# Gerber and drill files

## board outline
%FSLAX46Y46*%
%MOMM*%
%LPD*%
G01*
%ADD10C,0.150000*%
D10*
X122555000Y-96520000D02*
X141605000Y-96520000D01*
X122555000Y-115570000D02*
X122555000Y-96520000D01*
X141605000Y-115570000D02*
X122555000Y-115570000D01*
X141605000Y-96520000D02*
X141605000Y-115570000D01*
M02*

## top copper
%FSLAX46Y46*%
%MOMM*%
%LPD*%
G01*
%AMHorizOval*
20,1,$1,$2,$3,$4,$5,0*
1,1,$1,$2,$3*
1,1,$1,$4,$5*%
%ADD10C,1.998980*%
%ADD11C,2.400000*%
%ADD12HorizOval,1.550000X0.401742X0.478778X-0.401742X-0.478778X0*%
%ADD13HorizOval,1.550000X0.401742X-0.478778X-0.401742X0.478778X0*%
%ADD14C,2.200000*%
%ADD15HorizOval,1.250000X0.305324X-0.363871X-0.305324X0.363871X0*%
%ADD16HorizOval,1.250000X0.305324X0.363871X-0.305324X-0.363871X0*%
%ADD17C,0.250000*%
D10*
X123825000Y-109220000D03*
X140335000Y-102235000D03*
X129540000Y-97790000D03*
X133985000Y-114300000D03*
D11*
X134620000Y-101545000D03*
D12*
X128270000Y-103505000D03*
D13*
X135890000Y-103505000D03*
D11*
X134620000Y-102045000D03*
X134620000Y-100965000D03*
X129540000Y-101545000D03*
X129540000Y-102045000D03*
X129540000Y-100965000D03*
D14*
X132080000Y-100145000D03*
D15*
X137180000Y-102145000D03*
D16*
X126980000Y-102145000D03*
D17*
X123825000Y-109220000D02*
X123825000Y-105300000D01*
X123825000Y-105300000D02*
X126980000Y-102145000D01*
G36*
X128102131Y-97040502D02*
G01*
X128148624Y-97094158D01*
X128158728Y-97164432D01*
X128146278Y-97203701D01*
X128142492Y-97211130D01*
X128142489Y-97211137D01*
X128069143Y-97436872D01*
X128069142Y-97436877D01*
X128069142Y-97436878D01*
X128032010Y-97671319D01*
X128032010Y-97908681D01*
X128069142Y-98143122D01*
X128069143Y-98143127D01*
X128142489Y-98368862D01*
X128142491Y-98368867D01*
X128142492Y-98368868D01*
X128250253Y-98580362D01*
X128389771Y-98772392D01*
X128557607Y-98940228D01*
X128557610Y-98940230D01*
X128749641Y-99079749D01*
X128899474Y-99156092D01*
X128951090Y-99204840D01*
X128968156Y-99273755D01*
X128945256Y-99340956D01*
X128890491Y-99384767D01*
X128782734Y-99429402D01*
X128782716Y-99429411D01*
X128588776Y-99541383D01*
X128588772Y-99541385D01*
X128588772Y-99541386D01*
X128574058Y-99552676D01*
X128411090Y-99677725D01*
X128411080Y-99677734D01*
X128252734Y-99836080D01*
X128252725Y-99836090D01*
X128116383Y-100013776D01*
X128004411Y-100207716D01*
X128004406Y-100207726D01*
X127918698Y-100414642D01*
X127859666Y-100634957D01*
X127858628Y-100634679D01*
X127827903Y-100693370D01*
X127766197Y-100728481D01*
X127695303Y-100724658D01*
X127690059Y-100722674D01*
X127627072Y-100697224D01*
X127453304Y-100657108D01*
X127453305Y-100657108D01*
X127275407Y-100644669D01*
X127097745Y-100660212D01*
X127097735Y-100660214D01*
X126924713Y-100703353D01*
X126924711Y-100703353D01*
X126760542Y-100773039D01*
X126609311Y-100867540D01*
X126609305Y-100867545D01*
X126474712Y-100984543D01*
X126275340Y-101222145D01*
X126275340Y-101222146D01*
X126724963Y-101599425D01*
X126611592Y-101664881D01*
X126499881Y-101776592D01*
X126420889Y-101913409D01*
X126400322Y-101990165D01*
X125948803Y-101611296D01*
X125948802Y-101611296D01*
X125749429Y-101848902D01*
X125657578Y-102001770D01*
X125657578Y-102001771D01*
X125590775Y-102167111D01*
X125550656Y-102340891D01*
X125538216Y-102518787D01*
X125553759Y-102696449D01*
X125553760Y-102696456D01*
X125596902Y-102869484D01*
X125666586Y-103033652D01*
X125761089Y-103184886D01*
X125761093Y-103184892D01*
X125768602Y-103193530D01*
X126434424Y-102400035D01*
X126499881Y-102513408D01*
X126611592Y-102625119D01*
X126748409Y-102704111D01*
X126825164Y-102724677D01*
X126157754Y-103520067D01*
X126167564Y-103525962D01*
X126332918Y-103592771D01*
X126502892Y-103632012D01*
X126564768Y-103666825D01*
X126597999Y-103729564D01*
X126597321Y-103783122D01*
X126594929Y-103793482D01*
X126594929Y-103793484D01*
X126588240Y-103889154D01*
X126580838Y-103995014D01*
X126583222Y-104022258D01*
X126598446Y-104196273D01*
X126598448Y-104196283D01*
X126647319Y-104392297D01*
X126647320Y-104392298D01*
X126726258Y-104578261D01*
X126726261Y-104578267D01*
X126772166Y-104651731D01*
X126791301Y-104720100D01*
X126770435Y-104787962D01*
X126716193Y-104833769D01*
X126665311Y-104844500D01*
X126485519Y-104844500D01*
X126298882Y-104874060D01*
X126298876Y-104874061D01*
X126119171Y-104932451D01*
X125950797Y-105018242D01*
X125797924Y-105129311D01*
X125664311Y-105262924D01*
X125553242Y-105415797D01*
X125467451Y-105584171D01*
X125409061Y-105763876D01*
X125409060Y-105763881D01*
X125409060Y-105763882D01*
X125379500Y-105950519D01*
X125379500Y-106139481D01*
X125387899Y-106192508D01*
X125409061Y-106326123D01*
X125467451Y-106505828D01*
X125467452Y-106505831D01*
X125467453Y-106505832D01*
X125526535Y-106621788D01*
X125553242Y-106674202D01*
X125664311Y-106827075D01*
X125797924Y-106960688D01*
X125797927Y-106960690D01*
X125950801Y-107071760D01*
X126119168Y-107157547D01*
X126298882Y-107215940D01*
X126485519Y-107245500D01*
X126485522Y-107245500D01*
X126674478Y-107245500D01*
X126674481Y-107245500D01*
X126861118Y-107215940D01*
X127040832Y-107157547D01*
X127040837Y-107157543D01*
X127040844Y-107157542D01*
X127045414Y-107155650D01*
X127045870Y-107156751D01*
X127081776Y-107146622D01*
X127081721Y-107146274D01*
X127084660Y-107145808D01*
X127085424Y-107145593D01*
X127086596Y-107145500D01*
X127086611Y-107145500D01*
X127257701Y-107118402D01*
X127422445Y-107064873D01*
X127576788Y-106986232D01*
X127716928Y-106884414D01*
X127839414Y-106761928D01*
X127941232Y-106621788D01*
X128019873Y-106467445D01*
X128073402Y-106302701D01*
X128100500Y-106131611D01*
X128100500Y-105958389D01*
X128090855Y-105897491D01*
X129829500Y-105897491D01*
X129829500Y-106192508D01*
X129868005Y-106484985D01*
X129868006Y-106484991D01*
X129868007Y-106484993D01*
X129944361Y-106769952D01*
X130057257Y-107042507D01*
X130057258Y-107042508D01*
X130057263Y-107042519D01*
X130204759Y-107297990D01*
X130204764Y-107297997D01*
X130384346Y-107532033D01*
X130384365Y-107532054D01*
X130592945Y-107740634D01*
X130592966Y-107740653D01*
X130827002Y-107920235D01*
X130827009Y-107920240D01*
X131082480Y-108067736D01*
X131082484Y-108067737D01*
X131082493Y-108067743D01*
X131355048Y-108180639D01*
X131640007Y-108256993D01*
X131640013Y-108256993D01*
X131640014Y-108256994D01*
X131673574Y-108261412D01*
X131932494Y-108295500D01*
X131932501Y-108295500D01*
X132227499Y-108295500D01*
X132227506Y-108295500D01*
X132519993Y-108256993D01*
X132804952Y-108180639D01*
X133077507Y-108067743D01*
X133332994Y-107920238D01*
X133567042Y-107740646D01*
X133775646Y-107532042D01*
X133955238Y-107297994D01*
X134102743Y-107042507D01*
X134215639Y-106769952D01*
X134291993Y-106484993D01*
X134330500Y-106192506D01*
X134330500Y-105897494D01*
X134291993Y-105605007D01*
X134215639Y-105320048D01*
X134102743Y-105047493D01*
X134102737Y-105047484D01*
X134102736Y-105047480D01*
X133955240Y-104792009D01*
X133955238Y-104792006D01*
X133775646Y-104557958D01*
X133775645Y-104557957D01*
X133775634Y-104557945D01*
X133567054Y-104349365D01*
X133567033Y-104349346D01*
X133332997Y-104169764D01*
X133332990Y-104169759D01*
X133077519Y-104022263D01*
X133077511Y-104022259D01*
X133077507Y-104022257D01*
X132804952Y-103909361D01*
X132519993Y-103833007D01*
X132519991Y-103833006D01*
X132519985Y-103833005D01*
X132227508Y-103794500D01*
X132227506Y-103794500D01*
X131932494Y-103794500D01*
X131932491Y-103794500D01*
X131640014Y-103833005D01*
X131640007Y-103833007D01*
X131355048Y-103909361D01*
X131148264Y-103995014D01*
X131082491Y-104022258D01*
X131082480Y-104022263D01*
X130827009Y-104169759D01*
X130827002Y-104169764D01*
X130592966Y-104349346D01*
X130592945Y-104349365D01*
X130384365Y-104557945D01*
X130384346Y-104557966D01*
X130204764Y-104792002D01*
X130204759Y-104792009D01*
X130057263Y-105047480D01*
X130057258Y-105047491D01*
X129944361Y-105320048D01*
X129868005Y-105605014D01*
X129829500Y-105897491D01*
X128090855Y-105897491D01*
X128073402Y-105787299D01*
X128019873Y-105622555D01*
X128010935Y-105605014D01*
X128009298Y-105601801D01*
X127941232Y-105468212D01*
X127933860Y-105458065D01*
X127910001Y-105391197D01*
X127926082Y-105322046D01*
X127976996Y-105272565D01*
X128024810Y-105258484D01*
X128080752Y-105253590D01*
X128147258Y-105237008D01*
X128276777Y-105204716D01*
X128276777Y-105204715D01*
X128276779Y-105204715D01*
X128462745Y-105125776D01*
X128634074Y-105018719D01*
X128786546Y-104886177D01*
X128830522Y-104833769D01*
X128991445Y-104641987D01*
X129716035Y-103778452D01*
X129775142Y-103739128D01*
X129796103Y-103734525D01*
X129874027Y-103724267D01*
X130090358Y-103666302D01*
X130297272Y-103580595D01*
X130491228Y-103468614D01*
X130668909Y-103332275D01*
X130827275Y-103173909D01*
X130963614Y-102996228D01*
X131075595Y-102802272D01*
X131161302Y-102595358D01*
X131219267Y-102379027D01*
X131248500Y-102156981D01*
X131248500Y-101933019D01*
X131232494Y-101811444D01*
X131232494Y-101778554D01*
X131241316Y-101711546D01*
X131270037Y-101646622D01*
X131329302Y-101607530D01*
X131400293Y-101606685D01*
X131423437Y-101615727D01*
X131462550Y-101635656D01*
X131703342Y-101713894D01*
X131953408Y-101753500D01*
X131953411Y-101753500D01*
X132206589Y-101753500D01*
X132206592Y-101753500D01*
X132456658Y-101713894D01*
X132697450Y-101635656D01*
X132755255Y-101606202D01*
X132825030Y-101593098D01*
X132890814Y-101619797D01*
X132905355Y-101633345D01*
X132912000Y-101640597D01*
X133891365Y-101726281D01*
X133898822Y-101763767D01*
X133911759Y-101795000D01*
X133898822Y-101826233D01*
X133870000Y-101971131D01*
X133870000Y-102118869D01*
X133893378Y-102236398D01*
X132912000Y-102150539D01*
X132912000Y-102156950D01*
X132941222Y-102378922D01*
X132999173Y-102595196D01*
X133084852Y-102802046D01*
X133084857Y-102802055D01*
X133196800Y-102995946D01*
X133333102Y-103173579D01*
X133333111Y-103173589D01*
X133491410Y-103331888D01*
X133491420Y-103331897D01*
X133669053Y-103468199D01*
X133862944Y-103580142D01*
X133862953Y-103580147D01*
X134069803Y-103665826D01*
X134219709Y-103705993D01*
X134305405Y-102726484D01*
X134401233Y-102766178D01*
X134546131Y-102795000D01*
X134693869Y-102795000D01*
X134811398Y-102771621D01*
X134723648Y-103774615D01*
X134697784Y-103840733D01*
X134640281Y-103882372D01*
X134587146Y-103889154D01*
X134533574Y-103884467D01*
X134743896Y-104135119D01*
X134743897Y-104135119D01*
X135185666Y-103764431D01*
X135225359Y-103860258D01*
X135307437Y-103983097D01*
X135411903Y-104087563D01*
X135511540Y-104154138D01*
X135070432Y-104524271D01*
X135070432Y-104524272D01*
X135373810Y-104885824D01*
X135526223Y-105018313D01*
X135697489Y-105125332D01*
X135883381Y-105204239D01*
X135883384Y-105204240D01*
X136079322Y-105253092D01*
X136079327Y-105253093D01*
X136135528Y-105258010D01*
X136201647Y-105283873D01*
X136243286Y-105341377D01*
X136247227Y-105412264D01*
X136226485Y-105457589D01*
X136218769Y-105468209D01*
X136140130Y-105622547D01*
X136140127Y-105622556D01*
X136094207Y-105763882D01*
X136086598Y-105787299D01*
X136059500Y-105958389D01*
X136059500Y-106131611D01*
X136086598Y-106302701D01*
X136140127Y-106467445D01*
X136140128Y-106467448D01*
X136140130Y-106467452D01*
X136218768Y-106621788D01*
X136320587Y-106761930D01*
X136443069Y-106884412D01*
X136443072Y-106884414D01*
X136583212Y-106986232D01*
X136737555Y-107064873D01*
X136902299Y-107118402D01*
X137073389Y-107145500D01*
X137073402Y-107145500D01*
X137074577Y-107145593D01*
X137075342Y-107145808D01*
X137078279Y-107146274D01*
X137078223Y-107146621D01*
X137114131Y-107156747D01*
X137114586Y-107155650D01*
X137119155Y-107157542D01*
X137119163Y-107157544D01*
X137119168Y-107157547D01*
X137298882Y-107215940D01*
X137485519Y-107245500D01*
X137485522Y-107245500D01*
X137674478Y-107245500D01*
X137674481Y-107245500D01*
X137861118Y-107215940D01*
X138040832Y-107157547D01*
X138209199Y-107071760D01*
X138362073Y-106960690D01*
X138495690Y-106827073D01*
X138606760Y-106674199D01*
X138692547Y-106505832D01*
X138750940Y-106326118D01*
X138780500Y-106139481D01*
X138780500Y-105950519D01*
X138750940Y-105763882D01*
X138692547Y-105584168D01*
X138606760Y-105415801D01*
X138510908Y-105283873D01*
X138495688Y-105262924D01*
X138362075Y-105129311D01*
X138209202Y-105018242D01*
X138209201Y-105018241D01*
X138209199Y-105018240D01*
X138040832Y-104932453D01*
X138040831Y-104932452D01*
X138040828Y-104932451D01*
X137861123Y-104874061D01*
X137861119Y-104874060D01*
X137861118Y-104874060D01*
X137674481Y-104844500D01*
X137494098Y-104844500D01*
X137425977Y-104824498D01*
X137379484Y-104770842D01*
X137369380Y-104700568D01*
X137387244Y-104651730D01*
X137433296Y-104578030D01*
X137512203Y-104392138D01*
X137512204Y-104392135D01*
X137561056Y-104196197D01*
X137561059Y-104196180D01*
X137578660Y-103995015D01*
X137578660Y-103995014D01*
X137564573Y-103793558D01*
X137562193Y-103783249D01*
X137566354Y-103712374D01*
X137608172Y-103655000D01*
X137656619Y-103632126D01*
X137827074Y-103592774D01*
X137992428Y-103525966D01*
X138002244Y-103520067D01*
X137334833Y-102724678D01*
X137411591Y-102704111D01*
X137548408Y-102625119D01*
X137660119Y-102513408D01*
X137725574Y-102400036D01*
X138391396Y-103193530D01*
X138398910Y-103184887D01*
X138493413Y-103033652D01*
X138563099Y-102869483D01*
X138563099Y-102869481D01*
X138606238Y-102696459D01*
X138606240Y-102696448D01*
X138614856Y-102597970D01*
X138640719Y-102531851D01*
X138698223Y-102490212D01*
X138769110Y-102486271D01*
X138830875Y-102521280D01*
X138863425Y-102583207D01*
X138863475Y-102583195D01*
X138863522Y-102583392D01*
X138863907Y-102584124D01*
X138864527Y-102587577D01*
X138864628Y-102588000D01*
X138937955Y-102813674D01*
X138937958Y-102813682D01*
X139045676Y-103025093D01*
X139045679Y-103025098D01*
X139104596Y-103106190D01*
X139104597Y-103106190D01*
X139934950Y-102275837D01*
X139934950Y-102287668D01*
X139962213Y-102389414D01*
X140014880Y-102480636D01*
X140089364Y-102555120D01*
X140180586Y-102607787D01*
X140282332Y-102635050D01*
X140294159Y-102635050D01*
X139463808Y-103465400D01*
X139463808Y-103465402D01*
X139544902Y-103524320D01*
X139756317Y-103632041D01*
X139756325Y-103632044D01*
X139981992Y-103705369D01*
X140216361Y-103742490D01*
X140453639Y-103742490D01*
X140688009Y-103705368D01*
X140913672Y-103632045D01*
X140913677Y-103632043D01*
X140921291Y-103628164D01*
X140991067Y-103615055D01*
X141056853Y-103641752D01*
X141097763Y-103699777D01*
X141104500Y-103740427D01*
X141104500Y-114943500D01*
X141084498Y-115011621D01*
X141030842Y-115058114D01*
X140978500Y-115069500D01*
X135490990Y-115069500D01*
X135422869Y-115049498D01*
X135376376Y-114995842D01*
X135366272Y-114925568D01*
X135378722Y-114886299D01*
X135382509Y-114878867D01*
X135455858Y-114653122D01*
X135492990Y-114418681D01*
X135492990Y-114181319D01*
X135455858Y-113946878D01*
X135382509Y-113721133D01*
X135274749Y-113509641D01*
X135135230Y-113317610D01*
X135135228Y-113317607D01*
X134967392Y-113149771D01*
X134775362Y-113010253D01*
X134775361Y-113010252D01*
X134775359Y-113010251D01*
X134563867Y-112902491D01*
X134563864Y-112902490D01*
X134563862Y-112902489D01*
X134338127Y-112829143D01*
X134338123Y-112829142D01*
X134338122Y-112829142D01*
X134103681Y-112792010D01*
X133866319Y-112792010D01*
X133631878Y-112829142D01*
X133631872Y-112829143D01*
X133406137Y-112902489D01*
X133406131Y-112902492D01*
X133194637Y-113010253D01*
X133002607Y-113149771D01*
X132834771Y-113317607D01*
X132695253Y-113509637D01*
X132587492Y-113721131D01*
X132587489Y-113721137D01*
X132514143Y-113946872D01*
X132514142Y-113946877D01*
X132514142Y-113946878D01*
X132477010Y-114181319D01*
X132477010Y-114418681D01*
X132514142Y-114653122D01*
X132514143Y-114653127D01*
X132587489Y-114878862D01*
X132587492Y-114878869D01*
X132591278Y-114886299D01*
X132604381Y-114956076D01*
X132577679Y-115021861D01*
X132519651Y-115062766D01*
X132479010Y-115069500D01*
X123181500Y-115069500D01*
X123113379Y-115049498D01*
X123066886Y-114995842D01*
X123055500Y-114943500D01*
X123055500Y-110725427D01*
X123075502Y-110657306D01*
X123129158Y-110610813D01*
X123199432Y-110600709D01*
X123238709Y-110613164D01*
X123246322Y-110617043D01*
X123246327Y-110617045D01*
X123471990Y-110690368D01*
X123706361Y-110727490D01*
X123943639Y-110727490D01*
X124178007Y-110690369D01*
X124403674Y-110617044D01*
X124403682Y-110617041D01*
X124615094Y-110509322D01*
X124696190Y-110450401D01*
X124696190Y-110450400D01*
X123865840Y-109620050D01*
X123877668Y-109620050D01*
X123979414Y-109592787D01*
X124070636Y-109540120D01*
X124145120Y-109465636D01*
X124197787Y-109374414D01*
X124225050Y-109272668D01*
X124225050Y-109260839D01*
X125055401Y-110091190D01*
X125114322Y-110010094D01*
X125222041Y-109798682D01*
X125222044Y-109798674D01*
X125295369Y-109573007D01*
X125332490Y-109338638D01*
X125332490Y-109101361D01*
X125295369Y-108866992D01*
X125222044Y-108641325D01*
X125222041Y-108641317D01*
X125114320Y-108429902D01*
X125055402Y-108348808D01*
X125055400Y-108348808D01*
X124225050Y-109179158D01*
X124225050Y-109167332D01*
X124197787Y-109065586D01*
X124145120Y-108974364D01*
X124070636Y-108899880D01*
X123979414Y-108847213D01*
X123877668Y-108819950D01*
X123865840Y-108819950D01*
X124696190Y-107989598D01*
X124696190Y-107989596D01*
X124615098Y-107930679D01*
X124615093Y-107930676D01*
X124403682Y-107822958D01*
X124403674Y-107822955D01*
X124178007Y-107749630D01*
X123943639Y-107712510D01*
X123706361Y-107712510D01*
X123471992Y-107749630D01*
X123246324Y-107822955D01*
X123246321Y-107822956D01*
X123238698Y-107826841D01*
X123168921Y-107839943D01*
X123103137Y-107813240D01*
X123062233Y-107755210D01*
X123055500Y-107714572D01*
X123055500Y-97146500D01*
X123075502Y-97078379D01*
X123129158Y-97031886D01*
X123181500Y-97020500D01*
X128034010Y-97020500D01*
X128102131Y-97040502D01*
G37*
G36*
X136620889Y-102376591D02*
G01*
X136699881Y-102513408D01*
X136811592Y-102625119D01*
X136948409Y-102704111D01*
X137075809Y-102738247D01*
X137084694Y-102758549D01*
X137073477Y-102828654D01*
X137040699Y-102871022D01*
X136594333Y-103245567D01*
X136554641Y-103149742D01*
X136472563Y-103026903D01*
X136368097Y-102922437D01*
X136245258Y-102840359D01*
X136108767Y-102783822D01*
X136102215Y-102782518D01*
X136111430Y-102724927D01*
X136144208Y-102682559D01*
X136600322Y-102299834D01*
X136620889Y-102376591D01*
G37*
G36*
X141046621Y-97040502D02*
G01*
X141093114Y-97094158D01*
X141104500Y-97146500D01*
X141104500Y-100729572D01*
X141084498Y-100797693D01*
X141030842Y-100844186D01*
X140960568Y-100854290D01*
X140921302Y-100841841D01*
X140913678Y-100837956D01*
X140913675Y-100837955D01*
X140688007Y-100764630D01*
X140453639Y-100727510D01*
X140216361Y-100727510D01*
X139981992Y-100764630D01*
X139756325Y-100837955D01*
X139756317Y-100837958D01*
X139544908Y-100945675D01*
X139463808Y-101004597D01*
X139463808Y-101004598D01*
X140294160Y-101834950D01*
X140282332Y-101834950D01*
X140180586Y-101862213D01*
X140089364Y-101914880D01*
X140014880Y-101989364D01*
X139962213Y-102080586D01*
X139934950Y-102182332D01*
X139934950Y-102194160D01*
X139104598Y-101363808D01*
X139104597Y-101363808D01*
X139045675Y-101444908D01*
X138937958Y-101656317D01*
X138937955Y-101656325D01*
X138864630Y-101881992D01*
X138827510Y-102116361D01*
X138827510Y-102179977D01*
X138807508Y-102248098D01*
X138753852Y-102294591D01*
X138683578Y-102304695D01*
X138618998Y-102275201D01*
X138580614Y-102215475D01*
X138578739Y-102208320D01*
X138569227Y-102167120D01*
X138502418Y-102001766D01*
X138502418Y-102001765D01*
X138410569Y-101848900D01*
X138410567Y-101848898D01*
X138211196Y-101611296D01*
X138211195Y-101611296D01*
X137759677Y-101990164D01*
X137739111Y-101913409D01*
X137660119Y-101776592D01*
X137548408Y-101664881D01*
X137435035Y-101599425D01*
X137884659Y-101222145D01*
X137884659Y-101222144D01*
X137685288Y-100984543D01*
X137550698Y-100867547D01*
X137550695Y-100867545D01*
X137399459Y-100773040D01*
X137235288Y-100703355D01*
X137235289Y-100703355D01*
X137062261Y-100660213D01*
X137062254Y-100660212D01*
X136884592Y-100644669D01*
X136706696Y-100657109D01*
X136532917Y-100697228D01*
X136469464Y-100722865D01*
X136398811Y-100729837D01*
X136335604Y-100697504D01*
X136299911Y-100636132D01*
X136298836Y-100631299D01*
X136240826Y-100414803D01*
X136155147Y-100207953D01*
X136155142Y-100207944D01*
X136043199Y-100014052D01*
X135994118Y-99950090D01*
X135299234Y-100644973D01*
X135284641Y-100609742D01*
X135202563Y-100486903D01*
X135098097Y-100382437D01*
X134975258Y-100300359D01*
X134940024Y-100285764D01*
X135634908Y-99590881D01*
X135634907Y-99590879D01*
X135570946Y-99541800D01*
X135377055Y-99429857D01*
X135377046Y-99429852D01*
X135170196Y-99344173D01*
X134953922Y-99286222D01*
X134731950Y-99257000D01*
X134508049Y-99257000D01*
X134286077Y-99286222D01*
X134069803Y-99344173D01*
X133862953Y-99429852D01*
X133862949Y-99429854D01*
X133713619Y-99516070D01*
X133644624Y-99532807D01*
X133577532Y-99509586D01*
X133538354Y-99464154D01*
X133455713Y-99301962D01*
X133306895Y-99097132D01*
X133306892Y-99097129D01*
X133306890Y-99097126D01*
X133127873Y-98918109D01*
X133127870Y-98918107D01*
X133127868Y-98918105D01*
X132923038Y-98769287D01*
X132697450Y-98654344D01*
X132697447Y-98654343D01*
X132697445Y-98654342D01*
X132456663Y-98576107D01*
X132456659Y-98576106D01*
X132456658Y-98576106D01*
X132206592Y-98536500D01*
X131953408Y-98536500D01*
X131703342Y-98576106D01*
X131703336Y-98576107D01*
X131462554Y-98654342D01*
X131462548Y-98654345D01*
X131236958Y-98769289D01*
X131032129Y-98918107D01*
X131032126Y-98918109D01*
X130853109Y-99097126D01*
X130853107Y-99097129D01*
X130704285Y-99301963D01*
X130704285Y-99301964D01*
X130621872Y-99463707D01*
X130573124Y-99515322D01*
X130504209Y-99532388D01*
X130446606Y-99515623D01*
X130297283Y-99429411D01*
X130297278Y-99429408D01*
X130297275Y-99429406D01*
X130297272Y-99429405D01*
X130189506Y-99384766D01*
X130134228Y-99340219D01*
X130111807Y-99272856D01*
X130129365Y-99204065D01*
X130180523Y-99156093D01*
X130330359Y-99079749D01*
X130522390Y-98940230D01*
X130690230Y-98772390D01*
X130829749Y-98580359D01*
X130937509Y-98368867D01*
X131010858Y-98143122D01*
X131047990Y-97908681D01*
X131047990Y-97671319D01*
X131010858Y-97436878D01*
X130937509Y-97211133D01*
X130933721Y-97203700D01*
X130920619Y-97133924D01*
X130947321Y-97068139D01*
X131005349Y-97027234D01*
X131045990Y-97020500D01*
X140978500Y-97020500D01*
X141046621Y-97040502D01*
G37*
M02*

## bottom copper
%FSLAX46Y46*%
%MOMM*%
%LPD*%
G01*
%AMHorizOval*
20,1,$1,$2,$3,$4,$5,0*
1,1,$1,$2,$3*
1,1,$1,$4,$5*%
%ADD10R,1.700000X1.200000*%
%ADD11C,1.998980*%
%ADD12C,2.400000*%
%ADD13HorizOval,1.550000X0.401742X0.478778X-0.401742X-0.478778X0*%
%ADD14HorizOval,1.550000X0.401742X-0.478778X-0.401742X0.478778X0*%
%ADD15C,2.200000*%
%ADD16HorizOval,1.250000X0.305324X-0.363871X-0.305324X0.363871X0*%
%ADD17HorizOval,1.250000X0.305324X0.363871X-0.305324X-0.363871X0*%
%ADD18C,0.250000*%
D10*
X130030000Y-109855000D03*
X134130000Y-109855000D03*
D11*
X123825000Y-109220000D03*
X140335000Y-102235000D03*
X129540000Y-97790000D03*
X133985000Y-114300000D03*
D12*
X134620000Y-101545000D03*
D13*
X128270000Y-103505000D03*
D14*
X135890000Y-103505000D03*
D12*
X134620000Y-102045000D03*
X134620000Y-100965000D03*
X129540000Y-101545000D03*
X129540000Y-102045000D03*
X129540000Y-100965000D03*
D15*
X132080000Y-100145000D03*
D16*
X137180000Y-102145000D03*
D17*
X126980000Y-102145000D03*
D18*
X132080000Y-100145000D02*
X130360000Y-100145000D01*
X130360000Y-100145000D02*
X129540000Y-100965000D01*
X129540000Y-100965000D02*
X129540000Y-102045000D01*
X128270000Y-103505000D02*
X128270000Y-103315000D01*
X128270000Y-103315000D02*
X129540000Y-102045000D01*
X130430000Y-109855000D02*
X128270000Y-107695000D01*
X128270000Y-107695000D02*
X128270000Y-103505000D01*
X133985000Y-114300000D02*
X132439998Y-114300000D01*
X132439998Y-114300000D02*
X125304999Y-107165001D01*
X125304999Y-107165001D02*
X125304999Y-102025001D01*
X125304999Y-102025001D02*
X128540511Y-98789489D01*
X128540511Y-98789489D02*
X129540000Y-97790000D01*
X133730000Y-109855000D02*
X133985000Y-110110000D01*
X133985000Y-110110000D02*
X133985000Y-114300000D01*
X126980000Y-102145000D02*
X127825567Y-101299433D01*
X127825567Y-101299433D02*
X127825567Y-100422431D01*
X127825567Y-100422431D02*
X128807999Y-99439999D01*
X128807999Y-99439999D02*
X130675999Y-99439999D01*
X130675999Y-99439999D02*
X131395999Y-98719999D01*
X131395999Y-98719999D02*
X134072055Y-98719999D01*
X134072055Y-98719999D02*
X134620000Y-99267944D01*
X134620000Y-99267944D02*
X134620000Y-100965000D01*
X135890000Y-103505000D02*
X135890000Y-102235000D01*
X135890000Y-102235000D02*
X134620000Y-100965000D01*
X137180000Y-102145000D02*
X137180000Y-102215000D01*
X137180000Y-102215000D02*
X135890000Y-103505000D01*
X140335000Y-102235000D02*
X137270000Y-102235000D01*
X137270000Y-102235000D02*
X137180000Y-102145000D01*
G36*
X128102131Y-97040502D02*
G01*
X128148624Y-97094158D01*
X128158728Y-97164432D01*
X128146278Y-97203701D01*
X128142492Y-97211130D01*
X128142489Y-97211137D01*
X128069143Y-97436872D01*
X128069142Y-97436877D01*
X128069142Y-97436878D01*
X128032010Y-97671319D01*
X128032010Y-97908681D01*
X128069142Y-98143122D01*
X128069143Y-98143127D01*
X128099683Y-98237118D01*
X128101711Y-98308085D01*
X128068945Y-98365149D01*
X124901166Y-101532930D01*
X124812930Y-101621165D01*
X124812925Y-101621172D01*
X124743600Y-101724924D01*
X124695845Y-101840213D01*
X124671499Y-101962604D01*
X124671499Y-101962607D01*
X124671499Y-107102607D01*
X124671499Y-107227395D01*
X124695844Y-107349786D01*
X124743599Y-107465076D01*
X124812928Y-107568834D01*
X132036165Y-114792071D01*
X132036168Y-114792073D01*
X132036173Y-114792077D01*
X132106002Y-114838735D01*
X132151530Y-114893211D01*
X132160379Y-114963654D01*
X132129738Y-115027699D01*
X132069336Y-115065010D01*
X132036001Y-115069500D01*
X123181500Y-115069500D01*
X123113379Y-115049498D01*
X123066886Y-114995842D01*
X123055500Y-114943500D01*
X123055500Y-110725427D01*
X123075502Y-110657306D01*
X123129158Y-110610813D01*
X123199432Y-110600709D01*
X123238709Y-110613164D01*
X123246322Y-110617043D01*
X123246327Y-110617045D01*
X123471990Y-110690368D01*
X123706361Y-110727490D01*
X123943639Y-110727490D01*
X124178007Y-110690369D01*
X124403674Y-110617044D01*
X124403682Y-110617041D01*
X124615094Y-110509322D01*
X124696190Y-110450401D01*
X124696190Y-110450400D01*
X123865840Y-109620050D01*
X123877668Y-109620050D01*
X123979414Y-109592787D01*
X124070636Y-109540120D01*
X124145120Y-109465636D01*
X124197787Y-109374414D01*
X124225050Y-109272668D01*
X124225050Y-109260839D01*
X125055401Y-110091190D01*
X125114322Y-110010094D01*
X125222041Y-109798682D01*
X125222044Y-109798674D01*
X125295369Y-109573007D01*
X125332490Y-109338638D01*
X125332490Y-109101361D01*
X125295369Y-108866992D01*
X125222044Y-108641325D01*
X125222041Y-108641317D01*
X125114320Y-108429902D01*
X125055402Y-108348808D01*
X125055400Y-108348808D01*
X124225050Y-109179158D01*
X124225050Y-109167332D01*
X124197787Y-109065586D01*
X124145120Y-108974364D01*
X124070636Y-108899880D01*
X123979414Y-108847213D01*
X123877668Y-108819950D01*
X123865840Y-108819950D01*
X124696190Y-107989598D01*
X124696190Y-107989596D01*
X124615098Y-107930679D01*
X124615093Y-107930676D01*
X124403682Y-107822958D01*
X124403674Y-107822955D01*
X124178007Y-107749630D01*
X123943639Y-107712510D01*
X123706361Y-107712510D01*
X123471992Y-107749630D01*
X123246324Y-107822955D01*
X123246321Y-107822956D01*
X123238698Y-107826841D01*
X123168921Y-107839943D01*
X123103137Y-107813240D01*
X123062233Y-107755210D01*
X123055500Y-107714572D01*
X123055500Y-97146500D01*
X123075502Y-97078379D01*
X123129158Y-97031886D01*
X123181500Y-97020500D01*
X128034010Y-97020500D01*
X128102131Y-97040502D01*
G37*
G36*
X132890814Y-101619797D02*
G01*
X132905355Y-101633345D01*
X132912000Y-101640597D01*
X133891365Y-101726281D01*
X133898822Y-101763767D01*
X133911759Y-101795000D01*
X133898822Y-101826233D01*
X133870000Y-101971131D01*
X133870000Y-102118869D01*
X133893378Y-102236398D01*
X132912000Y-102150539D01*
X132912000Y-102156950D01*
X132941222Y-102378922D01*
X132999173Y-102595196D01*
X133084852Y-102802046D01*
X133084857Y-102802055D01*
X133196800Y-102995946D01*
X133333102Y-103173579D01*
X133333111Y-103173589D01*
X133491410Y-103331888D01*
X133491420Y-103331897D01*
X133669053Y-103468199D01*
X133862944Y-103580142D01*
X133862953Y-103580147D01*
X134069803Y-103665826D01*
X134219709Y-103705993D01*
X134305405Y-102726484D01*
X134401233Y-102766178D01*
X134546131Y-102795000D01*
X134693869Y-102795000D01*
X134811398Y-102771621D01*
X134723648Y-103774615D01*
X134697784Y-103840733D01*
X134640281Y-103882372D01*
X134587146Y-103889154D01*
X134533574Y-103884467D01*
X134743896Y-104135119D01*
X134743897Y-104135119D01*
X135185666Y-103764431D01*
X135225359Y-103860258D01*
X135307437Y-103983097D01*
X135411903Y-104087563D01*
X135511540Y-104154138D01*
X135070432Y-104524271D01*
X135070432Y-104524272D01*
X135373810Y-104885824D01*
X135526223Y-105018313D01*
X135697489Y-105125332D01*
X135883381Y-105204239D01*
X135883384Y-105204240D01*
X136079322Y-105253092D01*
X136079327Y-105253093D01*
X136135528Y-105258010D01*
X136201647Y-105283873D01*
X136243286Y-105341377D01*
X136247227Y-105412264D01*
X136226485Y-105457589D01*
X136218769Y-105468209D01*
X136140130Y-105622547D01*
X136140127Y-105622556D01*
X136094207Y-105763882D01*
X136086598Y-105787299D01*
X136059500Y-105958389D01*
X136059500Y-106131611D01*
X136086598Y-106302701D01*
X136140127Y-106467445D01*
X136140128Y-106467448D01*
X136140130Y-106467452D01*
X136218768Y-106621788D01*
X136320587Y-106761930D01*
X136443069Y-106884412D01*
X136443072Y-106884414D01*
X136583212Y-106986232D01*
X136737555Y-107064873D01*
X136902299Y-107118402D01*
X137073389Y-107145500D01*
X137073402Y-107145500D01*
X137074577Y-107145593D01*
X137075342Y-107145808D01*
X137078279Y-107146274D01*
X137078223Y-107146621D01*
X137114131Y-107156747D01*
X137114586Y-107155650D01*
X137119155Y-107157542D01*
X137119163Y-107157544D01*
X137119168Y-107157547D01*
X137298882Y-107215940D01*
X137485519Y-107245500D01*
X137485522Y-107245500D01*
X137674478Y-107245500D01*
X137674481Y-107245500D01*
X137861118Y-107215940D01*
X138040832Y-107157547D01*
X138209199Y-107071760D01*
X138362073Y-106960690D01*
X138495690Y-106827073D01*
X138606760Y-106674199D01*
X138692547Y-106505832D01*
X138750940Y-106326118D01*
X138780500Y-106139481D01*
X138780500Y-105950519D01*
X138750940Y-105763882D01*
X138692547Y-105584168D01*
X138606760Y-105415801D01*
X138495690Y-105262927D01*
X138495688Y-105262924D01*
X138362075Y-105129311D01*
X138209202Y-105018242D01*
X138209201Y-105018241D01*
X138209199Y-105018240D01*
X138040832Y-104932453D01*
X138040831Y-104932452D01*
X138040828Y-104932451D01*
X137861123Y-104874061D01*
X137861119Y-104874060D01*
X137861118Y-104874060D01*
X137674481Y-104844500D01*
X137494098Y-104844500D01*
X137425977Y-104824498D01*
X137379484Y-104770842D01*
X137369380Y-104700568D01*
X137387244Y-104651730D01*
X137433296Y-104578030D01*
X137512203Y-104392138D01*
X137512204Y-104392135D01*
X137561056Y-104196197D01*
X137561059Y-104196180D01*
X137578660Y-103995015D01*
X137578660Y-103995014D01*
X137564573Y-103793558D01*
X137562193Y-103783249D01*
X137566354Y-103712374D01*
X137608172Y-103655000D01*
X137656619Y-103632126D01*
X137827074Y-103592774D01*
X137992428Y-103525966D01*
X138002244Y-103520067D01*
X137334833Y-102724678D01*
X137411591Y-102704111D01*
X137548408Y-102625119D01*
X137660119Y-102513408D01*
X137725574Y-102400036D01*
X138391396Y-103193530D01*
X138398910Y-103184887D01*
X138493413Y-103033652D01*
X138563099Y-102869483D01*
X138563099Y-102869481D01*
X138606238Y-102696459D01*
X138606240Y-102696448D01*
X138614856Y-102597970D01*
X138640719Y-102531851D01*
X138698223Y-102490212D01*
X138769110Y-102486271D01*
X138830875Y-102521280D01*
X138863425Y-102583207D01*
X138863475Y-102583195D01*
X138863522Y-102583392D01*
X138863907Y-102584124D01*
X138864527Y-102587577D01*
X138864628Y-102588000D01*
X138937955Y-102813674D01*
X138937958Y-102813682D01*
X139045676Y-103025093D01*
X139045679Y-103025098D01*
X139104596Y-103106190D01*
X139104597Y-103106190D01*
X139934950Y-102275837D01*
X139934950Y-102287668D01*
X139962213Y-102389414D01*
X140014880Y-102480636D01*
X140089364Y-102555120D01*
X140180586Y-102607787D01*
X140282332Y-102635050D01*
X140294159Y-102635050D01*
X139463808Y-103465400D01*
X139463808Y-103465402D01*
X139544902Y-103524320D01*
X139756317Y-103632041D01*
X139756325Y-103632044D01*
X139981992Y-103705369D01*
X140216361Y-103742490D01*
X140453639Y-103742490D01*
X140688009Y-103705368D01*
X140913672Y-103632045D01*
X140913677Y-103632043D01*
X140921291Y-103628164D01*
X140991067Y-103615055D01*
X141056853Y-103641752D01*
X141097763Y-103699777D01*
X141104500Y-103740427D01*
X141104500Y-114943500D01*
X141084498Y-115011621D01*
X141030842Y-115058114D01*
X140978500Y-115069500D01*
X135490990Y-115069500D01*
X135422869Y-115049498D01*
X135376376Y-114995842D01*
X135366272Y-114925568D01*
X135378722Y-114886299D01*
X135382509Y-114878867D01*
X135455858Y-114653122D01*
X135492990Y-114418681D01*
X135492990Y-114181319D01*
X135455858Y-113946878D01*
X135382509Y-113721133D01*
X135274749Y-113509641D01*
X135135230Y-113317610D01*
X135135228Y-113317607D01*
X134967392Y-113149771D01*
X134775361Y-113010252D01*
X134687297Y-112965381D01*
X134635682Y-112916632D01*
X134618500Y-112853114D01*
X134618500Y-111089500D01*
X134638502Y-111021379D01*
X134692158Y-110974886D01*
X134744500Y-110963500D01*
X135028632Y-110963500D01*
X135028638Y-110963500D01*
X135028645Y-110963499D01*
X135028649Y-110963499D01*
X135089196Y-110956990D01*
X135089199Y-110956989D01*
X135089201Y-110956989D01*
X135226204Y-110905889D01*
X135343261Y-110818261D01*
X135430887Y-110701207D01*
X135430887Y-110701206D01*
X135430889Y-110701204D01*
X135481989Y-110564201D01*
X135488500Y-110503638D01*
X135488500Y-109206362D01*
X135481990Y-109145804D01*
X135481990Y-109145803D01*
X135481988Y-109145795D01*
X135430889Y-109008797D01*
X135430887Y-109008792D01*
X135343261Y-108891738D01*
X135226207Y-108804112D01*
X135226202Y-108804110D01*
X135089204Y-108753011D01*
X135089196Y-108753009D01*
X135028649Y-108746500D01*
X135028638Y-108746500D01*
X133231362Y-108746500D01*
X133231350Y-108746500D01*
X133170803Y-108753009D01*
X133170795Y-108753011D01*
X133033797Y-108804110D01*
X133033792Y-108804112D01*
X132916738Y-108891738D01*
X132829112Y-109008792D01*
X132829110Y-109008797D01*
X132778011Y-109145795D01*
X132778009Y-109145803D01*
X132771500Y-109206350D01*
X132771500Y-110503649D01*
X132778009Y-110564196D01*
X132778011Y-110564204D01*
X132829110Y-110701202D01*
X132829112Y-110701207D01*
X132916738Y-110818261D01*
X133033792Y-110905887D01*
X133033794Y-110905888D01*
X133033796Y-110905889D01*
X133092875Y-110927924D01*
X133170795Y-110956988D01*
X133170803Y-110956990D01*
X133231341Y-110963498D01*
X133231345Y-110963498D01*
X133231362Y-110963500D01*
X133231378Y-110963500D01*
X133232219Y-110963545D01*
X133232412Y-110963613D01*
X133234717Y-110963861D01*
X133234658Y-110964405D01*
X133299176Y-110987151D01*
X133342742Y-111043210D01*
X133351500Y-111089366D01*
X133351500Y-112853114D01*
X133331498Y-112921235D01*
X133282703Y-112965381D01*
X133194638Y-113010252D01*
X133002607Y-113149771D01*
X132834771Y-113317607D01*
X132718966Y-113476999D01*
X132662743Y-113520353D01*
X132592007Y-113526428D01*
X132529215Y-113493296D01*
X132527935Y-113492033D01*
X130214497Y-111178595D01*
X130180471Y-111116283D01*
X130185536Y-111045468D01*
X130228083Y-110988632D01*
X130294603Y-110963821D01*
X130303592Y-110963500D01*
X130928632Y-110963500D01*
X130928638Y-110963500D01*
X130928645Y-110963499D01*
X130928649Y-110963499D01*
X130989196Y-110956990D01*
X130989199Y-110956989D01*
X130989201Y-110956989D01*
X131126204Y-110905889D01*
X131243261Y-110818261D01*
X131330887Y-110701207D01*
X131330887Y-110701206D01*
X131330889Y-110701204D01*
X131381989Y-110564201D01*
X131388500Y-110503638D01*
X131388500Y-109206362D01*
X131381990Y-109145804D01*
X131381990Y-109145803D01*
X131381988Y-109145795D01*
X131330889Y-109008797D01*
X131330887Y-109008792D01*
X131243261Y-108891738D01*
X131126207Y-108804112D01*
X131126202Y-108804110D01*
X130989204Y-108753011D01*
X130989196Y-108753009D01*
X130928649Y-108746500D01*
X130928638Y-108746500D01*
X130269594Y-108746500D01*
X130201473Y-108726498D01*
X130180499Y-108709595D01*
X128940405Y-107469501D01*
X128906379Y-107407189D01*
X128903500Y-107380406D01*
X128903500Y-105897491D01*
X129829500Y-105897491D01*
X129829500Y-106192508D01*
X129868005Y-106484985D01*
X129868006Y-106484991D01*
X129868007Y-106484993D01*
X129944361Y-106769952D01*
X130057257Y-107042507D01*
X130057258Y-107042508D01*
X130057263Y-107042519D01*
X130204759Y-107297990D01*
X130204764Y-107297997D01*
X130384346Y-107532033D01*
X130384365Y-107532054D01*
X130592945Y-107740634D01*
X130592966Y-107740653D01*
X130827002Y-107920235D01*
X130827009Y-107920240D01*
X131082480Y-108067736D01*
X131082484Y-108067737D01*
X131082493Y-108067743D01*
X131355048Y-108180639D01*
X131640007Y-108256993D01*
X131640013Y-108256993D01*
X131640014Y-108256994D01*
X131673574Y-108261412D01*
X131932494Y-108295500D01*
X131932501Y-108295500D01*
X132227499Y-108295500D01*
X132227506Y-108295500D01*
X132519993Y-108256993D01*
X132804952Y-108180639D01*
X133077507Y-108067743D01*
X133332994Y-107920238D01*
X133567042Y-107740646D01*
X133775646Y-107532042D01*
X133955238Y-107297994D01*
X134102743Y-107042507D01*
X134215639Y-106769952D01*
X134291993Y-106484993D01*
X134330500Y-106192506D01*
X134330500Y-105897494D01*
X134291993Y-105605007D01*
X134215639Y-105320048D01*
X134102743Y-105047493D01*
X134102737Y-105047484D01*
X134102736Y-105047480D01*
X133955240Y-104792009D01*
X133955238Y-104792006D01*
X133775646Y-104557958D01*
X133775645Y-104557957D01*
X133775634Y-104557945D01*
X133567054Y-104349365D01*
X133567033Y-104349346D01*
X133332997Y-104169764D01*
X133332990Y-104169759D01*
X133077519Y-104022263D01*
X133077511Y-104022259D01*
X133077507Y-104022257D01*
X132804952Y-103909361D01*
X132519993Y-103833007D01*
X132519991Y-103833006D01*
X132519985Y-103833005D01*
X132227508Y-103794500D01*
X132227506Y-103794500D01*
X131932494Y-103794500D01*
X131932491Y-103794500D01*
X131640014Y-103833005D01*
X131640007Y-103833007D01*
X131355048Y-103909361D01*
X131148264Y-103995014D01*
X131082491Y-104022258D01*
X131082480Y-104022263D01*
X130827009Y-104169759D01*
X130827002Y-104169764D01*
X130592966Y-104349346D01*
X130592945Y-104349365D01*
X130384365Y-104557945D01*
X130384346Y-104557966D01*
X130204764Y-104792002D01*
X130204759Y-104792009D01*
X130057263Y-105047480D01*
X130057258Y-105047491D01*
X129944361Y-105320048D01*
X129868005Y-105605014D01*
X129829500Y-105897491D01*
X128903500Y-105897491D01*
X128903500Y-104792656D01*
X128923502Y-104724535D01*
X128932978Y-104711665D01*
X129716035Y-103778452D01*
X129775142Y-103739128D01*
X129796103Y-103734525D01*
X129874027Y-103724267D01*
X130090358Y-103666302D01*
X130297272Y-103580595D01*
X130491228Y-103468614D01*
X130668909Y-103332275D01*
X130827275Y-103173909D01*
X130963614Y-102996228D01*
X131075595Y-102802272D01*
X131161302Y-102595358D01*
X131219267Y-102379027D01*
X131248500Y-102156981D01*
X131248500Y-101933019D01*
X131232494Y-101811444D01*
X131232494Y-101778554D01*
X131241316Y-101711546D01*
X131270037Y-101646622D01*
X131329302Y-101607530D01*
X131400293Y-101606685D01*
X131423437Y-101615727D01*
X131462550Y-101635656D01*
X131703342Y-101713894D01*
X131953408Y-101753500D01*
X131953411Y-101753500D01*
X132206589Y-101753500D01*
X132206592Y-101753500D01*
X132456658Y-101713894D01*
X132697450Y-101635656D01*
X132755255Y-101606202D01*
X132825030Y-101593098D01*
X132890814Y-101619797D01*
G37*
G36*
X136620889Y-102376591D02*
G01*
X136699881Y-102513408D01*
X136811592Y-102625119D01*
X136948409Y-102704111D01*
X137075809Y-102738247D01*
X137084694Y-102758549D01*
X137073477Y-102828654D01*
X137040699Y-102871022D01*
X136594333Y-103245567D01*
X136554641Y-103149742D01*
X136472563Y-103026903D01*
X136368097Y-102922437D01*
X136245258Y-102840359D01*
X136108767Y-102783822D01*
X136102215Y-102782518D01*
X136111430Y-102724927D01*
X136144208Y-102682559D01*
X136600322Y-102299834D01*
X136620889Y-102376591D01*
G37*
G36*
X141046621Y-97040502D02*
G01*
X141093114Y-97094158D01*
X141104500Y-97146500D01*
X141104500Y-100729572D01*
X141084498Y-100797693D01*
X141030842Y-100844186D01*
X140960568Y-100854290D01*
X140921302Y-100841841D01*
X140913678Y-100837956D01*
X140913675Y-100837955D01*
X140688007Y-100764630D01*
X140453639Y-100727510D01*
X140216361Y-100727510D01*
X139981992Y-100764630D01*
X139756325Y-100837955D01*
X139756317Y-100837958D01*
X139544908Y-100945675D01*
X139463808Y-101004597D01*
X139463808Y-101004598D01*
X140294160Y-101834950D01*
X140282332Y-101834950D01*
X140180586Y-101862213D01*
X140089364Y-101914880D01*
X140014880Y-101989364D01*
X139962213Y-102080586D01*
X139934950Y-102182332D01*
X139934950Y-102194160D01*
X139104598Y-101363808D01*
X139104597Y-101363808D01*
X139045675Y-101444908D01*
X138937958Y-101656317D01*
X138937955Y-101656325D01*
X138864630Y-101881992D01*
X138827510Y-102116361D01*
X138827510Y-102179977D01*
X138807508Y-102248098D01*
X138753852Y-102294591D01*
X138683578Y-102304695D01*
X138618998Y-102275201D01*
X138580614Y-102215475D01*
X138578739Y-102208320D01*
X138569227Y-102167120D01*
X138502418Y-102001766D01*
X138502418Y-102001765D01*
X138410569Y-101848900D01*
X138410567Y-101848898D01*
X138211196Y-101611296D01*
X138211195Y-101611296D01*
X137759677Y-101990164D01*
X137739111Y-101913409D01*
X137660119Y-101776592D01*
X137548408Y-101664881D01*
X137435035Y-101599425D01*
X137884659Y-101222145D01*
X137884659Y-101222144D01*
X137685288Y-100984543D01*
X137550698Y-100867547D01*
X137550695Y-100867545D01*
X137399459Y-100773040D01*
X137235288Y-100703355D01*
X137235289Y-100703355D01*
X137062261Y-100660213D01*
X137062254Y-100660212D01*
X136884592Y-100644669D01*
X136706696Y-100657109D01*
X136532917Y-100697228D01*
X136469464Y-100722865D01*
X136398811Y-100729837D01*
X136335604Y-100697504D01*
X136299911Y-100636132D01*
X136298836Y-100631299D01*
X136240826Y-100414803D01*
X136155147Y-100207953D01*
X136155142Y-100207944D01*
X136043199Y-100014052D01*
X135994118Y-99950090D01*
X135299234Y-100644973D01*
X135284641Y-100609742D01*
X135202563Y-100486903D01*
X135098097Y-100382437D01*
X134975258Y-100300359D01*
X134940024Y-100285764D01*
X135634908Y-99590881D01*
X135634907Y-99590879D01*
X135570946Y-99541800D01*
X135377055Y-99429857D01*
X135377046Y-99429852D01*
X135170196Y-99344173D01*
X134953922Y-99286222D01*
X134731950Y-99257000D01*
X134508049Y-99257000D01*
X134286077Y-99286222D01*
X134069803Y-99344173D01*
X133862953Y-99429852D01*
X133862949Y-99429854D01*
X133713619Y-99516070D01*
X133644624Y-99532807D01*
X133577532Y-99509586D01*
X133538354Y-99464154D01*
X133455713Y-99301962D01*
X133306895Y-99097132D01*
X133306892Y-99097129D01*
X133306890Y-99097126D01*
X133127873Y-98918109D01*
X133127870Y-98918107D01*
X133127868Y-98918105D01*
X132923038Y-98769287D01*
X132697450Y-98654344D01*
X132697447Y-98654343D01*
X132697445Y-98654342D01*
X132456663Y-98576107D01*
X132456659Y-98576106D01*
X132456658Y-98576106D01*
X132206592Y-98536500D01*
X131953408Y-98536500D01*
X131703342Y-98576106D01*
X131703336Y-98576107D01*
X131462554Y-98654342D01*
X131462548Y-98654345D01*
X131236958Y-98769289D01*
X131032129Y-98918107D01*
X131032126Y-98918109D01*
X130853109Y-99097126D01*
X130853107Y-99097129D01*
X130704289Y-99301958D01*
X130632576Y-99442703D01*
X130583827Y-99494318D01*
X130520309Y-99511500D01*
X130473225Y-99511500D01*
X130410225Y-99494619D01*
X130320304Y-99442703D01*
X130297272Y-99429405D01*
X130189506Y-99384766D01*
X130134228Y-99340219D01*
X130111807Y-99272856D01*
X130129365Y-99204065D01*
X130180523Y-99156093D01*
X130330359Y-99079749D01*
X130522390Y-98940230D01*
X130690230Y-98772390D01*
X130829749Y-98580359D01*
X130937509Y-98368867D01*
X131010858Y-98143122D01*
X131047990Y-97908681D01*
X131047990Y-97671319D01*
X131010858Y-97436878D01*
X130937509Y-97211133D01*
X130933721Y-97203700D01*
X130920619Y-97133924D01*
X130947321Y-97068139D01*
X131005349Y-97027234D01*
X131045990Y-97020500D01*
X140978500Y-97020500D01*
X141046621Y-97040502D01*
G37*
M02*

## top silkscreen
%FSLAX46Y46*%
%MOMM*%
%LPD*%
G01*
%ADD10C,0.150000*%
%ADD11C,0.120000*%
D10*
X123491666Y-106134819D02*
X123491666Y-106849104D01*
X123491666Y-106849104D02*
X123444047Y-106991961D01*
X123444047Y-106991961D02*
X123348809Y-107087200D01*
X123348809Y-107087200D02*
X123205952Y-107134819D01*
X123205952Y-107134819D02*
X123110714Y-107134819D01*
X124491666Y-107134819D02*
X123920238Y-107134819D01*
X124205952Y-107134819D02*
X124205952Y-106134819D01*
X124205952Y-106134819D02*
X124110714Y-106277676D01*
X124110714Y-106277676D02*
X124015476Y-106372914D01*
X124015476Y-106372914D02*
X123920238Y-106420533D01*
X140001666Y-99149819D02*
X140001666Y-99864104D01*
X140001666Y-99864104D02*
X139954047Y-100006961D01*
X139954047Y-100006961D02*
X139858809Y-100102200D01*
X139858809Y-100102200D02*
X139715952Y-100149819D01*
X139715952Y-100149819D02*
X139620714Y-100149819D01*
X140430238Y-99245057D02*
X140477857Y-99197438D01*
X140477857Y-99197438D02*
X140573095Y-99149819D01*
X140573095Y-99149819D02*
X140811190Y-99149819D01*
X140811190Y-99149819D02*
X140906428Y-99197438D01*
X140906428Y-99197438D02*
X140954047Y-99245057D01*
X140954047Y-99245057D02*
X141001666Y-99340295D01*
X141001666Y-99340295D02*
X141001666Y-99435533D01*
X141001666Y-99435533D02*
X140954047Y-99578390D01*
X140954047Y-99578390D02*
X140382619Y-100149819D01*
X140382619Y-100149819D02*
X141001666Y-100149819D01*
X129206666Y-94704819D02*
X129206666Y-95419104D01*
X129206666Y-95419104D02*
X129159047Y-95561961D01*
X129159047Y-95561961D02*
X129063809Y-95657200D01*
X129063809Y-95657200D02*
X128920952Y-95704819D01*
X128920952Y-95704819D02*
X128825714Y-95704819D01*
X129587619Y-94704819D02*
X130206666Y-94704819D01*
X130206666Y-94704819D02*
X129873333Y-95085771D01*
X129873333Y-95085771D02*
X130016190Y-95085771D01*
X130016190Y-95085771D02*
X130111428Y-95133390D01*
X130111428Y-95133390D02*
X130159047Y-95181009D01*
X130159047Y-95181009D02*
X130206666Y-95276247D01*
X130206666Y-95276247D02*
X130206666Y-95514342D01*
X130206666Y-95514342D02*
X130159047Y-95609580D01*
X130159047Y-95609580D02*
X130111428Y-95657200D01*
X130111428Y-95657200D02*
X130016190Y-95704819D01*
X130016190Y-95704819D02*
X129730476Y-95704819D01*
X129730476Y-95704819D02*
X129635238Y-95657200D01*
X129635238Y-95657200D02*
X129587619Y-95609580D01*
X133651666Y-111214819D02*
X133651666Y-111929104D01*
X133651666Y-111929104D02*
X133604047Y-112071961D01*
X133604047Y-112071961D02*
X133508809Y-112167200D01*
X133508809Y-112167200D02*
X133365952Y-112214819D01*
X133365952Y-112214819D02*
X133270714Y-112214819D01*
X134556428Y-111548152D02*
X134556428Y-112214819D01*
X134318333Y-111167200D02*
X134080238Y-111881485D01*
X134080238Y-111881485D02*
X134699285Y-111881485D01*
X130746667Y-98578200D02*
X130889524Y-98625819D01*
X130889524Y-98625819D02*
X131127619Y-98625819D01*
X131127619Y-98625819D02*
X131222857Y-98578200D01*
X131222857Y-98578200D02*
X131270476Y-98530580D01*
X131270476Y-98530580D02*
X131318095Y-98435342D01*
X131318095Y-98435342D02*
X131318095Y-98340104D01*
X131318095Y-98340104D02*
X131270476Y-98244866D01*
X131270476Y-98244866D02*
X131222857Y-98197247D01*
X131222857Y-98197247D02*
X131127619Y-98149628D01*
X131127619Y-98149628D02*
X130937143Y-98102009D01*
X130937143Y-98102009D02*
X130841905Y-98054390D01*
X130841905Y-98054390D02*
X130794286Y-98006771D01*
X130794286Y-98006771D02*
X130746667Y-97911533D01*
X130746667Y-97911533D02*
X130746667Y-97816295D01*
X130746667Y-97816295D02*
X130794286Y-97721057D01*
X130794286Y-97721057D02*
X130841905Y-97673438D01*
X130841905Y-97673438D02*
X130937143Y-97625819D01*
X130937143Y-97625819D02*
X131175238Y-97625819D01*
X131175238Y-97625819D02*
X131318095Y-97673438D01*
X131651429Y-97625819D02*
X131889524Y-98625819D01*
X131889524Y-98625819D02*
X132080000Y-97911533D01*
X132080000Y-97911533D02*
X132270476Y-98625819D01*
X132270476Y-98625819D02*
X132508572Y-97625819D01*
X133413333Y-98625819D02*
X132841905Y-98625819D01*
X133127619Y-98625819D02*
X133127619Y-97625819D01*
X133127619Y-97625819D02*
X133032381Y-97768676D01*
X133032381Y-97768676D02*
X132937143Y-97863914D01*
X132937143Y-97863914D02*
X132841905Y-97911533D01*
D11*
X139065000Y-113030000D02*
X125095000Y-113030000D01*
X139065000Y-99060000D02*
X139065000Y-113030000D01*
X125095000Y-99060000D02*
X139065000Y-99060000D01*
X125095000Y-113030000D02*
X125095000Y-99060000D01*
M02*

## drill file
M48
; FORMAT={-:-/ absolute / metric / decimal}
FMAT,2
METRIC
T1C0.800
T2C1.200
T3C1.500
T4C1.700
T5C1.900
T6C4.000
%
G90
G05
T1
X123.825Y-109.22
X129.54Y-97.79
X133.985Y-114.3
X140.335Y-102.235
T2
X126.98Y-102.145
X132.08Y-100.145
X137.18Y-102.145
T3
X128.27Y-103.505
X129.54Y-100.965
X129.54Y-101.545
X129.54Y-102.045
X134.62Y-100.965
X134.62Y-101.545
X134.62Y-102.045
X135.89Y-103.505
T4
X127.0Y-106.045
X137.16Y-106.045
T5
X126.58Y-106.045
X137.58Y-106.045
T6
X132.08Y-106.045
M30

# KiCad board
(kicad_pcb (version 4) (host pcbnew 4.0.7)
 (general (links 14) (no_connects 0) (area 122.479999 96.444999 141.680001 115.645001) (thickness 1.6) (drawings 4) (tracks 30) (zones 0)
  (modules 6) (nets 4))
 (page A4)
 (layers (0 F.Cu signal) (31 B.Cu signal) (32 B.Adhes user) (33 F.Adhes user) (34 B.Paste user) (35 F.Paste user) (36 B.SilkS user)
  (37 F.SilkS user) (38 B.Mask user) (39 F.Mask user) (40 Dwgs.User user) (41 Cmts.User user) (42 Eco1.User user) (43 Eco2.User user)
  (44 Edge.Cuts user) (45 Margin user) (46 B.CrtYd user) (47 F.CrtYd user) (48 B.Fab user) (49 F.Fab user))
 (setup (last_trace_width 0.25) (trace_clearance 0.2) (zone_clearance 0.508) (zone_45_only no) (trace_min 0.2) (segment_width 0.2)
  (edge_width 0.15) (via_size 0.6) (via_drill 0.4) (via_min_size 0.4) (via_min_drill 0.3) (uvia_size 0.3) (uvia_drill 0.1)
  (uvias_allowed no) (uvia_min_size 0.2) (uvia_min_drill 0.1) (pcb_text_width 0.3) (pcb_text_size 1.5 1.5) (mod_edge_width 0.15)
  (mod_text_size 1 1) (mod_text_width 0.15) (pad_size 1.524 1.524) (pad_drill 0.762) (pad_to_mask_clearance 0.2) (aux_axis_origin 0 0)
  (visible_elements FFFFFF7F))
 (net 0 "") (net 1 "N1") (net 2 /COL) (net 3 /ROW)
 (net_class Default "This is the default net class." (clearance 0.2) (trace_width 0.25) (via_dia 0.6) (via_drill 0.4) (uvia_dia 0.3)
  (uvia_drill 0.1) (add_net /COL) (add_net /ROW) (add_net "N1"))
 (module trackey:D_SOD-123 (layer B.Cu) (at 132.08 109.855)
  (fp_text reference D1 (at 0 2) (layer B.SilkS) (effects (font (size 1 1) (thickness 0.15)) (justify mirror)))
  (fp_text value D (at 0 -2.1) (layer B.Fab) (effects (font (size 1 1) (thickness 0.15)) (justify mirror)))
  (pad 1 smd rect (at -1.65 0) (size 1.7 1.2) (drill (offset -0.4 0)) (layers B.Cu B.Paste B.Mask) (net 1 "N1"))
  (pad 2 smd rect (at 1.65 0) (size 1.7 1.2) (drill (offset 0.4 0)) (layers B.Cu B.Paste B.Mask) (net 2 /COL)))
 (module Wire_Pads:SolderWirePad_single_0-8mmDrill (layer F.Cu) (at 123.825 109.22)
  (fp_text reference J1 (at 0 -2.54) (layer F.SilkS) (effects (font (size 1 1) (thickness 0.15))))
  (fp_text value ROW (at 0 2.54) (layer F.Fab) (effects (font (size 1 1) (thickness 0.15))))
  (pad 1 thru_hole circle (at 0 0) (size 1.99898 1.99898) (drill 0.8001) (layers *.Cu *.Mask) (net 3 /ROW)))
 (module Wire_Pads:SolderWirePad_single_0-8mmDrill (layer F.Cu) (at 140.335 102.235)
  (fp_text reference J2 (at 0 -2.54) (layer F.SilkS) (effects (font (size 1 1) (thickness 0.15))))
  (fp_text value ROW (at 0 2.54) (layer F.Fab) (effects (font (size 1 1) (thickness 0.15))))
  (pad 1 thru_hole circle (at 0 0) (size 1.99898 1.99898) (drill 0.8001) (layers *.Cu *.Mask) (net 3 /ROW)))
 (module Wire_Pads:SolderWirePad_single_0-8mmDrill (layer F.Cu) (at 129.54 97.79)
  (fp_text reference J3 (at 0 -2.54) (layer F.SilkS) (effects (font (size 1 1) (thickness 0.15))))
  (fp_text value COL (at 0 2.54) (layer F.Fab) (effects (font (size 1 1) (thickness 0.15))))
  (pad 1 thru_hole circle (at 0 0) (size 1.99898 1.99898) (drill 0.8001) (layers *.Cu *.Mask) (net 2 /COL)))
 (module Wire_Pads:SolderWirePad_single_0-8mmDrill (layer F.Cu) (at 133.985 114.3)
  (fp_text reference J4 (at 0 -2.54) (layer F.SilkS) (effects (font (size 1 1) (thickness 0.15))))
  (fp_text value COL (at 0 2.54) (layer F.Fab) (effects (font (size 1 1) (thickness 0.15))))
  (pad 1 thru_hole circle (at 0 0) (size 1.99898 1.99898) (drill 0.8001) (layers *.Cu *.Mask) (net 2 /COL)))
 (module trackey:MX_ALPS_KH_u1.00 (layer F.Cu) (at 132.08 106.045)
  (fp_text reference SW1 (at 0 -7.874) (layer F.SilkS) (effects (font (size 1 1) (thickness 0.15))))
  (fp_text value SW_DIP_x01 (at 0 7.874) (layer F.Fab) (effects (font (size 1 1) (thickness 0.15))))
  (fp_line (start 6.985 6.985) (end -6.985 6.985) (layer F.SilkS) (width 0.12))
  (fp_line (start 6.985 -6.985) (end 6.985 6.985) (layer F.SilkS) (width 0.12))
  (fp_line (start -6.985 -6.985) (end 6.985 -6.985) (layer F.SilkS) (width 0.12))
  (fp_line (start -6.985 6.985) (end -6.985 -6.985) (layer F.SilkS) (width 0.12))
  (pad 1 thru_hole circle (at 2.54 -4.5) (size 2.4 2.4) (drill 1.5) (layers *.Cu *.Mask) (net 3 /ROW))
  (pad 2 thru_hole oval (at -3.81 -2.54 50) (size 2.8 1.55) (drill 1.5) (layers *.Cu *.Mask) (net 1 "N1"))
  (pad "" np_thru_hole circle (at 0 0) (size 4 4) (drill 4) (layers *.Cu *.Mask))
  (pad "" np_thru_hole circle (at -5.08 0) (size 1.7 1.7) (drill 1.7) (layers *.Cu *.Mask))
  (pad "" np_thru_hole circle (at 5.08 0) (size 1.7 1.7) (drill 1.7) (layers *.Cu *.Mask))
  (pad "" np_thru_hole circle (at -5.5 0) (size 1.9 1.9) (drill 1.9) (layers *.Cu *.Mask))
  (pad "" np_thru_hole circle (at 5.5 0) (size 1.9 1.9) (drill 1.9) (layers *.Cu *.Mask))
  (pad 1 thru_hole oval (at 3.81 -2.54 310) (size 2.8 1.55) (drill 1.5) (layers *.Cu *.Mask) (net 3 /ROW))
  (pad 1 thru_hole circle (at 2.54 -4 310) (size 2.4 2.4) (drill 1.5) (layers *.Cu *.Mask) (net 3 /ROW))
  (pad 1 thru_hole circle (at 2.54 -5.08) (size 2.4 2.4) (drill 1.5) (layers *.Cu *.Mask) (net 3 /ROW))
  (pad 2 thru_hole circle (at -2.54 -4.5) (size 2.4 2.4) (drill 1.5) (layers *.Cu *.Mask) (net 1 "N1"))
  (pad 2 thru_hole circle (at -2.54 -4) (size 2.4 2.4) (drill 1.5) (layers *.Cu *.Mask) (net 1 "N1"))
  (pad 2 thru_hole circle (at -2.54 -5.08) (size 2.4 2.4) (drill 1.5) (layers *.Cu *.Mask) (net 1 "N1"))
  (pad 2 thru_hole circle (at 0 -5.9) (size 2.2 2.2) (drill 1.2) (layers *.Cu *.Mask) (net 1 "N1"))
  (pad 1 thru_hole oval (at 5.1 -3.9 310) (size 2.2 1.25) (drill 1.2) (layers *.Cu *.Mask) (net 3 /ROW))
  (pad 1 thru_hole oval (at -5.1 -3.9 50) (size 2.2 1.25) (drill 1.2) (layers *.Cu *.Mask) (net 3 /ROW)))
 (gr_line (start 122.555 96.52) (end 141.605 96.52) (layer Edge.Cuts) (width 0.15))
 (gr_line (start 122.555 115.57) (end 122.555 96.52) (layer Edge.Cuts) (width 0.15))
 (gr_line (start 141.605 115.57) (end 122.555 115.57) (layer Edge.Cuts) (width 0.15))
 (gr_line (start 141.605 96.52) (end 141.605 115.57) (layer Edge.Cuts) (width 0.15))
 (segment (start 132.08 100.145) (end 130.36 100.145) (width 0.25) (layer B.Cu) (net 1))
 (segment (start 130.36 100.145) (end 129.54 100.965) (width 0.25) (layer B.Cu) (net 1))
 (segment (start 129.54 100.965) (end 129.54 102.045) (width 0.25) (layer B.Cu) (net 1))
 (segment (start 128.27 103.505) (end 128.27 103.315) (width 0.25) (layer B.Cu) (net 1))
 (segment (start 128.27 103.315) (end 129.54 102.045) (width 0.25) (layer B.Cu) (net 1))
 (segment (start 130.43 109.855) (end 128.27 107.695) (width 0.25) (layer B.Cu) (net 1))
 (segment (start 128.27 107.695) (end 128.27 103.505) (width 0.25) (layer B.Cu) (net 1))
 (segment (start 133.985 114.3) (end 132.439998 114.3) (width 0.25) (layer B.Cu) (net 2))
 (segment (start 132.439998 114.3) (end 125.304999 107.165001) (width 0.25) (layer B.Cu) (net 2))
 (segment (start 125.304999 107.165001) (end 125.304999 102.025001) (width 0.25) (layer B.Cu) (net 2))
 (segment (start 125.304999 102.025001) (end 128.540511 98.789489) (width 0.25) (layer B.Cu) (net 2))
 (segment (start 128.540511 98.789489) (end 129.54 97.79) (width 0.25) (layer B.Cu) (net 2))
 (segment (start 133.73 109.855) (end 133.985 110.11) (width 0.25) (layer B.Cu) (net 2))
 (segment (start 133.985 110.11) (end 133.985 114.3) (width 0.25) (layer B.Cu) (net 2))
 (segment (start 123.825 109.22) (end 123.825 105.3) (width 0.25) (layer F.Cu) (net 3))
 (segment (start 123.825 105.3) (end 126.98 102.145) (width 0.25) (layer F.Cu) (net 3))
 (segment (start 126.98 102.145) (end 127.825567 101.299433) (width 0.25) (layer B.Cu) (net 3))
 (segment (start 127.825567 101.299433) (end 127.825567 100.422431) (width 0.25) (layer B.Cu) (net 3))
 (segment (start 127.825567 100.422431) (end 128.807999 99.439999) (width 0.25) (layer B.Cu) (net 3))
 (segment (start 128.807999 99.439999) (end 130.675999 99.439999) (width 0.25) (layer B.Cu) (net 3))
 (segment (start 130.675999 99.439999) (end 131.395999 98.719999) (width 0.25) (layer B.Cu) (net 3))
 (segment (start 131.395999 98.719999) (end 134.072055 98.719999) (width 0.25) (layer B.Cu) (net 3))
 (segment (start 134.072055 98.719999) (end 134.62 99.267944) (width 0.25) (layer B.Cu) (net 3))
 (segment (start 134.62 99.267944) (end 134.62 100.965) (width 0.25) (layer B.Cu) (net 3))
 (segment (start 135.89 103.505) (end 135.89 102.235) (width 0.25) (layer B.Cu) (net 3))
 (segment (start 135.89 102.235) (end 134.62 100.965) (width 0.25) (layer B.Cu) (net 3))
 (segment (start 137.18 102.145) (end 137.18 102.215) (width 0.25) (layer B.Cu) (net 3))
 (segment (start 137.18 102.215) (end 135.89 103.505) (width 0.25) (layer B.Cu) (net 3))
 (segment (start 140.335 102.235) (end 137.27 102.235) (width 0.25) (layer B.Cu) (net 3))
 (segment (start 137.27 102.235) (end 137.18 102.145) (width 0.25) (layer B.Cu) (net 3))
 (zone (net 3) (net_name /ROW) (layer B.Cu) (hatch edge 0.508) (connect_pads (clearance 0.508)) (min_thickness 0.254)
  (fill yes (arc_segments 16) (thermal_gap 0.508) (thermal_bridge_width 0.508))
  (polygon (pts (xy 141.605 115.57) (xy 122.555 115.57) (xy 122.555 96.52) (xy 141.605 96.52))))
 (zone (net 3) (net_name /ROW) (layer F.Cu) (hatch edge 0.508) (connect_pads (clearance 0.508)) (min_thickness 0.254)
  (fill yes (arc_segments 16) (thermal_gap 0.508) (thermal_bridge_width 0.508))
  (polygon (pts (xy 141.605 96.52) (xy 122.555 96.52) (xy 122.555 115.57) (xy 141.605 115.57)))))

